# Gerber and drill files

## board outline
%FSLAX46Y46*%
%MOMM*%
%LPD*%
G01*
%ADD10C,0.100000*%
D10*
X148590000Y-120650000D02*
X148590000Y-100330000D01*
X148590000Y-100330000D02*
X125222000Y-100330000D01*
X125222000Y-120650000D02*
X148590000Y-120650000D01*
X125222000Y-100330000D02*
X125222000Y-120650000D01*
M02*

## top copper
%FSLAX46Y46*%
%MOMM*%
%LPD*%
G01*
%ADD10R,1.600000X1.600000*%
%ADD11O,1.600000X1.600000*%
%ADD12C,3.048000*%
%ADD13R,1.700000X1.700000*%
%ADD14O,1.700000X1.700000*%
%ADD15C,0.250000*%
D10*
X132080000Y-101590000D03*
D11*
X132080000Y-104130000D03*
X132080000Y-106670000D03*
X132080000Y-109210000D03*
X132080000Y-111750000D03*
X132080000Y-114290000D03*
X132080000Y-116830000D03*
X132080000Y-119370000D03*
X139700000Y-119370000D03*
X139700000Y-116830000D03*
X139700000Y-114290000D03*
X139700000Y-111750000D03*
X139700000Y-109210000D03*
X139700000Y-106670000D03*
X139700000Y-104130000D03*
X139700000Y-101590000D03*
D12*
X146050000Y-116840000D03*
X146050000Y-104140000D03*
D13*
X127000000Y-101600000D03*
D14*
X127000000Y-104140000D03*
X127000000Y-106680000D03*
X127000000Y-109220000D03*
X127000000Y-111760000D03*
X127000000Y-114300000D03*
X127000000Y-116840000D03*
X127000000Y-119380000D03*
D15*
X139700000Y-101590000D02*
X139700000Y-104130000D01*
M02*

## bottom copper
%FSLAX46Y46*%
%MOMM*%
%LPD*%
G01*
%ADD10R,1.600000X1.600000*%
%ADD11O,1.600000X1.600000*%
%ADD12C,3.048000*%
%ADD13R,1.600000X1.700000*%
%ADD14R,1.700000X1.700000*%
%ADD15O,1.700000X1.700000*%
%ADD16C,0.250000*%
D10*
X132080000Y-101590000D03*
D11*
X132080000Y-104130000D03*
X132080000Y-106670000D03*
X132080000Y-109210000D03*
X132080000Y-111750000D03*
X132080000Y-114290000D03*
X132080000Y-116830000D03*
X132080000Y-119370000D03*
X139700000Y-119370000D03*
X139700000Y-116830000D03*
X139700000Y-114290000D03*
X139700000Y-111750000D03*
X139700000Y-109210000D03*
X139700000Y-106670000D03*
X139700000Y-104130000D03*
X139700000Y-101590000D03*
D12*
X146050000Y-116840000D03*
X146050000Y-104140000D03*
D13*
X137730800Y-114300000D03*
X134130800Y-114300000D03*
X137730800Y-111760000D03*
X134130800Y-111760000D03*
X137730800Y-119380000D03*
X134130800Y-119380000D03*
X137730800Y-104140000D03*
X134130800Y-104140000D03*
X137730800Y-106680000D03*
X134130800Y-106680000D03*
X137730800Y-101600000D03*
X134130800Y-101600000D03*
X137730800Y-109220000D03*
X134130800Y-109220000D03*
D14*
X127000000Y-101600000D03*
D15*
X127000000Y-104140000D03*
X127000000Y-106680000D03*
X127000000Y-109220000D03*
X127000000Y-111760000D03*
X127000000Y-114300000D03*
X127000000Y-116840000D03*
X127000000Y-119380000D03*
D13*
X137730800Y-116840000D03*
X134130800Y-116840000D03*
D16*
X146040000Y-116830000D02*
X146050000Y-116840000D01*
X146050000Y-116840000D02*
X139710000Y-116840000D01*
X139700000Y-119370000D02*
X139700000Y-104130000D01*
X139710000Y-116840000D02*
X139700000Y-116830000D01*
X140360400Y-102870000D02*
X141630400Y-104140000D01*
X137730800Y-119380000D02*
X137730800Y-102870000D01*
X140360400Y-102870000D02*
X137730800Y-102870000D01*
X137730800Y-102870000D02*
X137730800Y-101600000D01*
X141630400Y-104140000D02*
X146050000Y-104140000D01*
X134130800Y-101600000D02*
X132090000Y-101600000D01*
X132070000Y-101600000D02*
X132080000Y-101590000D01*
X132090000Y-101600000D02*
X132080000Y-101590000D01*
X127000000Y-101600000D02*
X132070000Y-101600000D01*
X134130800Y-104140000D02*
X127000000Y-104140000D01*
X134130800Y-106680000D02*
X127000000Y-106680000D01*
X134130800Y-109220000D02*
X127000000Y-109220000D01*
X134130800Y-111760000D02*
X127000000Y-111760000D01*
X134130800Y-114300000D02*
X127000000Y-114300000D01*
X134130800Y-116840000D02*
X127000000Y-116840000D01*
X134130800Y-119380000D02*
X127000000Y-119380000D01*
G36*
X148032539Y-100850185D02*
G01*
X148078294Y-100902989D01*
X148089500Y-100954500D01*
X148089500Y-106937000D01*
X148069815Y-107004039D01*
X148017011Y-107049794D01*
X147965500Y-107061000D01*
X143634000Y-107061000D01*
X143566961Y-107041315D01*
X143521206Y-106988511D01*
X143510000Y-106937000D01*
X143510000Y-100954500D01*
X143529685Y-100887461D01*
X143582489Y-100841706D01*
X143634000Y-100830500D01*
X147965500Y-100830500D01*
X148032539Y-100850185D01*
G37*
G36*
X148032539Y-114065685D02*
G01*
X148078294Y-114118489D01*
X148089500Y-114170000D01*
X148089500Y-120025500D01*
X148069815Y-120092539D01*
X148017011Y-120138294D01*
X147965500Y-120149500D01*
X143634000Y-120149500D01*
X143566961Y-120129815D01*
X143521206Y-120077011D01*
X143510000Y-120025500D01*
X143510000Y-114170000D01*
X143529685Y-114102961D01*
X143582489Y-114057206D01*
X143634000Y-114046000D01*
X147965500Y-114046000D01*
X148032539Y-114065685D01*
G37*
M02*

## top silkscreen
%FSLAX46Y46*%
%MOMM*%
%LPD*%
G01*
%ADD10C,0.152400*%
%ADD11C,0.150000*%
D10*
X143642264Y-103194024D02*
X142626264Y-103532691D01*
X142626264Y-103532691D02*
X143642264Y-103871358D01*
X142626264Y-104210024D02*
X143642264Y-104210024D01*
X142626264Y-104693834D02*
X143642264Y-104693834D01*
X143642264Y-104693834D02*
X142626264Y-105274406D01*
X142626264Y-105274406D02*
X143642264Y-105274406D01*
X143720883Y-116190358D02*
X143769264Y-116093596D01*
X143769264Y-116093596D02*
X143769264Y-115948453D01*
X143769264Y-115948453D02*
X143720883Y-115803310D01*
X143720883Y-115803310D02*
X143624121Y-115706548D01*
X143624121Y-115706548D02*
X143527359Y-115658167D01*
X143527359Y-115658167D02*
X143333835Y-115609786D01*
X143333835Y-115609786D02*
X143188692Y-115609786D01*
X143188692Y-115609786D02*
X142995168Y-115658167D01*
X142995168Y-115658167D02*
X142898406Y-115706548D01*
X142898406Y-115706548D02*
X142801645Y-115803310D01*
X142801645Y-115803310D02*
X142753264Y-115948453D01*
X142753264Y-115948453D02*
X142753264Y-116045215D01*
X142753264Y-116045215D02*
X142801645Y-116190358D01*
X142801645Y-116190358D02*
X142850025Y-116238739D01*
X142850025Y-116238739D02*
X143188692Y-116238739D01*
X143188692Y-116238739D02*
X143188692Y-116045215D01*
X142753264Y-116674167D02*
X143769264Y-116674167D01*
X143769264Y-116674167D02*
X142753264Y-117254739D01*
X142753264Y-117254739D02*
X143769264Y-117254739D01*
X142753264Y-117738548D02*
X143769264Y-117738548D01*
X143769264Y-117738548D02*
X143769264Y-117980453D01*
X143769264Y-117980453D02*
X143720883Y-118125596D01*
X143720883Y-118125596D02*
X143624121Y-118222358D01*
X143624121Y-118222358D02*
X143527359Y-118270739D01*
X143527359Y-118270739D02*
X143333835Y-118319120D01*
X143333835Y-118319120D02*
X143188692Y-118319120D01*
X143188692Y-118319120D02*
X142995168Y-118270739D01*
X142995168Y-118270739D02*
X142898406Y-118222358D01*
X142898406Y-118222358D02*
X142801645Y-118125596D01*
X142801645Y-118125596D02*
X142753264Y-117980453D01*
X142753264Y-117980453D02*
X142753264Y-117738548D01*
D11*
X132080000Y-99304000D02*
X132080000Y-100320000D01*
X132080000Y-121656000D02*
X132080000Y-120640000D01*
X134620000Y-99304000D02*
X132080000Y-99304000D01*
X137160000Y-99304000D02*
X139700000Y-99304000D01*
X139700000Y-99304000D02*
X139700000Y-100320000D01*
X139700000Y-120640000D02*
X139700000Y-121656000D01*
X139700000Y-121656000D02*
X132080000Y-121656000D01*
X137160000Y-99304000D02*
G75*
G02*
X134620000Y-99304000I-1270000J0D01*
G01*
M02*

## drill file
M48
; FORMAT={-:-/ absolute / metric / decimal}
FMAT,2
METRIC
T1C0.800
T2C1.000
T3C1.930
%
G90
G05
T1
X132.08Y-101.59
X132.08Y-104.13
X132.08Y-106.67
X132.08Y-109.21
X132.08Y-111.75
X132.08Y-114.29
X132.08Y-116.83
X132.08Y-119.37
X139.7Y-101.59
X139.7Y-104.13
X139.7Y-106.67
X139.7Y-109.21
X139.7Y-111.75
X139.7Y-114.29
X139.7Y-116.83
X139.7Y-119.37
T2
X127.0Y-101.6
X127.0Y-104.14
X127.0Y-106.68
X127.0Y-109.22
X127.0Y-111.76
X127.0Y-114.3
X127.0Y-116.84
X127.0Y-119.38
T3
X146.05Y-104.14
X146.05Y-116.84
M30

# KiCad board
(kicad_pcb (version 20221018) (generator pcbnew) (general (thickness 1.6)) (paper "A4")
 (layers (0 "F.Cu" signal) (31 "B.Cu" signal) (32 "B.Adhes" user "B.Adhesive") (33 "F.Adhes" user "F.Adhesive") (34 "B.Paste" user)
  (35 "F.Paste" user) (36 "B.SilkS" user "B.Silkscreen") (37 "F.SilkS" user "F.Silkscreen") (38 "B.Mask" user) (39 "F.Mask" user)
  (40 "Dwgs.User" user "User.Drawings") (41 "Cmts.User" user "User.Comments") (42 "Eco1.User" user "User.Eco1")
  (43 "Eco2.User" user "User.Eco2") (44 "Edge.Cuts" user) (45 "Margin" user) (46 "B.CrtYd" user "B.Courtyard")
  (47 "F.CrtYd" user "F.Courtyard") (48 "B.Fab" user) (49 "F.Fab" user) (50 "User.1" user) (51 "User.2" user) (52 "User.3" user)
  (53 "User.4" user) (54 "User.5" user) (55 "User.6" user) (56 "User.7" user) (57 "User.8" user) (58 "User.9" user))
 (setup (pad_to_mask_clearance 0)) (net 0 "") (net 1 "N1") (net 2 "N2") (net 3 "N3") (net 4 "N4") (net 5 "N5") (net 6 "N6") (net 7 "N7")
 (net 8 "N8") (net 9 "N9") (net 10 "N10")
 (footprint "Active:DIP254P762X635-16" (layer "F.Cu") (at 132.08 101.59)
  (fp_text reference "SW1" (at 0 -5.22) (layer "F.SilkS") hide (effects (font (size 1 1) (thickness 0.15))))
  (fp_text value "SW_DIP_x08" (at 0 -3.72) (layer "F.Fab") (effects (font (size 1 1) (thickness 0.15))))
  (fp_line (start 0 -2.286) (end 0 -1.27) (stroke (width 0.15) (type solid)) (layer "F.SilkS"))
  (fp_line (start 0 20.066) (end 0 19.05) (stroke (width 0.15) (type solid)) (layer "F.SilkS"))
  (fp_line (start 2.54 -2.286) (end 0 -2.286) (stroke (width 0.15) (type solid)) (layer "F.SilkS"))
  (fp_line (start 5.08 -2.286) (end 7.62 -2.286) (stroke (width 0.15) (type solid)) (layer "F.SilkS"))
  (fp_line (start 7.62 -2.286) (end 7.62 -1.27) (stroke (width 0.15) (type solid)) (layer "F.SilkS"))
  (fp_line (start 7.62 19.05) (end 7.62 20.066) (stroke (width 0.15) (type solid)) (layer "F.SilkS"))
  (fp_line (start 7.62 20.066) (end 0 20.066) (stroke (width 0.15) (type solid)) (layer "F.SilkS"))
  (fp_arc (start 5.08 -2.286) (mid 3.81 -1.016) (end 2.54 -2.286) (stroke (width 0.15) (type solid)) (layer "F.SilkS"))
  (pad "1" thru_hole rect (at 0 0) (size 1.6 1.6) (drill 0.8) (layers "*.Cu" "*.Mask") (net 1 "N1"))
  (pad "2" thru_hole oval (at 0 2.54) (size 1.6 1.6) (drill 0.8) (layers "*.Cu" "*.Mask") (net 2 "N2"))
  (pad "3" thru_hole oval (at 0 5.08) (size 1.6 1.6) (drill 0.8) (layers "*.Cu" "*.Mask") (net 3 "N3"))
  (pad "4" thru_hole oval (at 0 7.62) (size 1.6 1.6) (drill 0.8) (layers "*.Cu" "*.Mask") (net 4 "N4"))
  (pad "5" thru_hole oval (at 0 10.16) (size 1.6 1.6) (drill 0.8) (layers "*.Cu" "*.Mask") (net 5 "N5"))
  (pad "6" thru_hole oval (at 0 12.7) (size 1.6 1.6) (drill 0.8) (layers "*.Cu" "*.Mask") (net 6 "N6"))
  (pad "7" thru_hole oval (at 0 15.24) (size 1.6 1.6) (drill 0.8) (layers "*.Cu" "*.Mask") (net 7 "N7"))
  (pad "8" thru_hole oval (at 0 17.78) (size 1.6 1.6) (drill 0.8) (layers "*.Cu" "*.Mask") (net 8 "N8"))
  (pad "9" thru_hole oval (at 7.62 17.78) (size 1.6 1.6) (drill 0.8) (layers "*.Cu" "*.Mask") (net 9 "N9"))
  (pad "10" thru_hole oval (at 7.62 15.24) (size 1.6 1.6) (drill 0.8) (layers "*.Cu" "*.Mask") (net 9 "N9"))
  (pad "11" thru_hole oval (at 7.62 12.7) (size 1.6 1.6) (drill 0.8) (layers "*.Cu" "*.Mask") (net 9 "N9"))
  (pad "12" thru_hole oval (at 7.62 10.16) (size 1.6 1.6) (drill 0.8) (layers "*.Cu" "*.Mask") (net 9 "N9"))
  (pad "13" thru_hole oval (at 7.62 7.62) (size 1.6 1.6) (drill 0.8) (layers "*.Cu" "*.Mask") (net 9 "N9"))
  (pad "14" thru_hole oval (at 7.62 5.08) (size 1.6 1.6) (drill 0.8) (layers "*.Cu" "*.Mask") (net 9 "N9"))
  (pad "15" thru_hole oval (at 7.62 2.54) (size 1.6 1.6) (drill 0.8) (layers "*.Cu" "*.Mask") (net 9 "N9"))
  (pad "16" thru_hole oval (at 7.62 0) (size 1.6 1.6) (drill 0.8) (layers "*.Cu" "*.Mask") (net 9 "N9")))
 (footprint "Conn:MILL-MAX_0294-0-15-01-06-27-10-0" (layer "F.Cu") (at 146.05 116.84)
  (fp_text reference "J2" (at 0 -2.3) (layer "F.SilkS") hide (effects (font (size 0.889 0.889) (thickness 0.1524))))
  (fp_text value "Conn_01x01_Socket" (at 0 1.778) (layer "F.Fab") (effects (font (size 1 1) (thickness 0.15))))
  (pad "1" thru_hole circle (at 0 0) (size 3.048 3.048) (drill 1.9304) (layers "*.Cu" "*.Mask") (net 9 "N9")))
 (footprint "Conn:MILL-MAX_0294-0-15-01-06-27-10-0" (layer "F.Cu") (at 146.05 104.14)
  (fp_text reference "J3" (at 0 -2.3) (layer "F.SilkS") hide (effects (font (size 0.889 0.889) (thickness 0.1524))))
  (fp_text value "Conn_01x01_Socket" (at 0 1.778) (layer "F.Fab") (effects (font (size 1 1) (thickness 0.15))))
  (pad "1" thru_hole circle (at 0 0) (size 3.048 3.048) (drill 1.9304) (layers "*.Cu" "*.Mask") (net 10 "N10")))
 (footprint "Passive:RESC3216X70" (layer "B.Cu") (at 135.9308 114.3 180)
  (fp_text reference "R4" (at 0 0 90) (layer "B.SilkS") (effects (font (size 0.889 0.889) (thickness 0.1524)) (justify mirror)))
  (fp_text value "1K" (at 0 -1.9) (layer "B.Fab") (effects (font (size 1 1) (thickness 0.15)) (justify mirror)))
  (pad "1" smd rect (at -1.8 0 180) (size 1.6 1.7) (layers "B.Cu" "B.Paste" "B.Mask") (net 10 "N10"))
  (pad "2" smd rect (at 1.8 0 180) (size 1.6 1.7) (layers "B.Cu" "B.Paste" "B.Mask") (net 6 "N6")))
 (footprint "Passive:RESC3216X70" (layer "B.Cu") (at 135.9308 111.76 180)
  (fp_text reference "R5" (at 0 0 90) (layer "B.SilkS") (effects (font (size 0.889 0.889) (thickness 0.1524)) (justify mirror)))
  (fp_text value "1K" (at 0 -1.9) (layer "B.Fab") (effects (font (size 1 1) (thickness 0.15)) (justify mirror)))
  (pad "1" smd rect (at -1.8 0 180) (size 1.6 1.7) (layers "B.Cu" "B.Paste" "B.Mask") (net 10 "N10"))
  (pad "2" smd rect (at 1.8 0 180) (size 1.6 1.7) (layers "B.Cu" "B.Paste" "B.Mask") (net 5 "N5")))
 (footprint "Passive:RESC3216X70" (layer "B.Cu") (at 135.9308 119.38 180)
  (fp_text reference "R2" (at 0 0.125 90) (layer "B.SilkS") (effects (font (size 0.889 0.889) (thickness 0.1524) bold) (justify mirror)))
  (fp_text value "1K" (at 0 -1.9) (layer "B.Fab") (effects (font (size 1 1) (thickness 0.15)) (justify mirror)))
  (pad "1" smd rect (at -1.8 0 180) (size 1.6 1.7) (layers "B.Cu" "B.Paste" "B.Mask") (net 10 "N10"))
  (pad "2" smd rect (at 1.8 0 180) (size 1.6 1.7) (layers "B.Cu" "B.Paste" "B.Mask") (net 8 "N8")))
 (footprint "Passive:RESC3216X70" (layer "B.Cu") (at 135.9308 104.14 180)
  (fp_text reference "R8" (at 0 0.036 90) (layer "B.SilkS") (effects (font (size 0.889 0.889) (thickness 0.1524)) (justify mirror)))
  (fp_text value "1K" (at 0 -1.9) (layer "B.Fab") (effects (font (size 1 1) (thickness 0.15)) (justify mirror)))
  (pad "1" smd rect (at -1.8 0 180) (size 1.6 1.7) (layers "B.Cu" "B.Paste" "B.Mask") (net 10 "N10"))
  (pad "2" smd rect (at 1.8 0 180) (size 1.6 1.7) (layers "B.Cu" "B.Paste" "B.Mask") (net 2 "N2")))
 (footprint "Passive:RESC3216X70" (layer "B.Cu") (at 135.9308 106.68 180)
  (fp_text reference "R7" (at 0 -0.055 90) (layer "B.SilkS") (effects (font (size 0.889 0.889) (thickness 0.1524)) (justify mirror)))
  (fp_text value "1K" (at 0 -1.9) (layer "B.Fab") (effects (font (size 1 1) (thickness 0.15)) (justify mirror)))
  (pad "1" smd rect (at -1.8 0 180) (size 1.6 1.7) (layers "B.Cu" "B.Paste" "B.Mask") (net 10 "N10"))
  (pad "2" smd rect (at 1.8 0 180) (size 1.6 1.7) (layers "B.Cu" "B.Paste" "B.Mask") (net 3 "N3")))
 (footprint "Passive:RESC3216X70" (layer "B.Cu") (at 135.9308 101.6 180)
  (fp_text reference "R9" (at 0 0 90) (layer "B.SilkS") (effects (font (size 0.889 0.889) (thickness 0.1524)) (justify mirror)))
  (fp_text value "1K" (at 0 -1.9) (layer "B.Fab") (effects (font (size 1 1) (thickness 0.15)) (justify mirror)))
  (pad "1" smd rect (at -1.8 0 180) (size 1.6 1.7) (layers "B.Cu" "B.Paste" "B.Mask") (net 10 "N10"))
  (pad "2" smd rect (at 1.8 0 180) (size 1.6 1.7) (layers "B.Cu" "B.Paste" "B.Mask") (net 1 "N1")))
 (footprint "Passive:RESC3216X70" (layer "B.Cu") (at 135.9308 109.22 180)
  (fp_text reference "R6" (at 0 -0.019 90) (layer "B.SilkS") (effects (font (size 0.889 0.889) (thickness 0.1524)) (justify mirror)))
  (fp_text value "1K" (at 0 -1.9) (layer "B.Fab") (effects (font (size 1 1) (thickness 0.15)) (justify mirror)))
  (pad "1" smd rect (at -1.8 0 180) (size 1.6 1.7) (layers "B.Cu" "B.Paste" "B.Mask") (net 10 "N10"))
  (pad "2" smd rect (at 1.8 0 180) (size 1.6 1.7) (layers "B.Cu" "B.Paste" "B.Mask") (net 4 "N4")))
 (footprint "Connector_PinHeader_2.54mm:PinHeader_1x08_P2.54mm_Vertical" (layer "B.Cu") (at 127 101.6 180)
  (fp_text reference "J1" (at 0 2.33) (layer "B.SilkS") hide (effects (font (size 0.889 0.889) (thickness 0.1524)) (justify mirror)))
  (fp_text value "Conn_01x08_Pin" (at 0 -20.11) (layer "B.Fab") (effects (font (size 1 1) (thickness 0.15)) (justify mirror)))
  (pad "1" thru_hole rect (at 0 0 180) (size 1.7 1.7) (drill 1) (layers "*.Cu" "*.Mask") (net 1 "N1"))
  (pad "2" thru_hole oval (at 0 -2.54 180) (size 1.7 1.7) (drill 1) (layers "*.Cu" "*.Mask") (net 2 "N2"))
  (pad "3" thru_hole oval (at 0 -5.08 180) (size 1.7 1.7) (drill 1) (layers "*.Cu" "*.Mask") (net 3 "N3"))
  (pad "4" thru_hole oval (at 0 -7.62 180) (size 1.7 1.7) (drill 1) (layers "*.Cu" "*.Mask") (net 4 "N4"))
  (pad "5" thru_hole oval (at 0 -10.16 180) (size 1.7 1.7) (drill 1) (layers "*.Cu" "*.Mask") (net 5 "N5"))
  (pad "6" thru_hole oval (at 0 -12.7 180) (size 1.7 1.7) (drill 1) (layers "*.Cu" "*.Mask") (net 6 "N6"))
  (pad "7" thru_hole oval (at 0 -15.24 180) (size 1.7 1.7) (drill 1) (layers "*.Cu" "*.Mask") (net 7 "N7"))
  (pad "8" thru_hole oval (at 0 -17.78 180) (size 1.7 1.7) (drill 1) (layers "*.Cu" "*.Mask") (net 8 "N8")))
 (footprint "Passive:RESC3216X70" (layer "B.Cu") (at 135.9308 116.84 180)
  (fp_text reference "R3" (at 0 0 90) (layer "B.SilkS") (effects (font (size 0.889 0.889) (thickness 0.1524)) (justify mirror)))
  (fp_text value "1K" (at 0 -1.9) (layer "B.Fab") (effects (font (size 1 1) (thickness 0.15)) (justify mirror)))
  (pad "1" smd rect (at -1.8 0 180) (size 1.6 1.7) (layers "B.Cu" "B.Paste" "B.Mask") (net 10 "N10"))
  (pad "2" smd rect (at 1.8 0 180) (size 1.6 1.7) (layers "B.Cu" "B.Paste" "B.Mask") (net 7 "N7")))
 (gr_line (start 148.59 120.65) (end 148.59 100.33) (stroke (width 0.1) (type default)) (layer "Edge.Cuts"))
 (gr_line (start 148.59 100.33) (end 125.222 100.33) (stroke (width 0.1) (type default)) (layer "Edge.Cuts"))
 (gr_line (start 125.222 120.65) (end 148.59 120.65) (stroke (width 0.1) (type default)) (layer "Edge.Cuts"))
 (gr_line (start 125.222 100.33) (end 125.222 120.65) (stroke (width 0.1) (type default)) (layer "Edge.Cuts"))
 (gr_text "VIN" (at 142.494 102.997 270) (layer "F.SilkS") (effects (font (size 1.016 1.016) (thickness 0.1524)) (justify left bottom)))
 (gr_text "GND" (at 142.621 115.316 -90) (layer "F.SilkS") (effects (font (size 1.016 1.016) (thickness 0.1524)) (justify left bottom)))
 (segment (start 139.7 101.59) (end 139.7 104.13) (width 0.25) (layer "F.Cu") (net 9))
 (segment (start 146.04 116.83) (end 146.05 116.84) (width 0.25) (layer "B.Cu") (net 9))
 (segment (start 146.05 116.84) (end 139.71 116.84) (width 0.25) (layer "B.Cu") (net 9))
 (segment (start 139.7 119.37) (end 139.7 104.13) (width 0.25) (layer "B.Cu") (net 9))
 (segment (start 139.71 116.84) (end 139.7 116.83) (width 0.25) (layer "B.Cu") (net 9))
 (segment (start 140.3604 102.87) (end 141.6304 104.14) (width 0.25) (layer "B.Cu") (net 10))
 (segment (start 137.7308 119.38) (end 137.7308 102.87) (width 0.25) (layer "B.Cu") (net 10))
 (segment (start 140.3604 102.87) (end 137.7308 102.87) (width 0.25) (layer "B.Cu") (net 10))
 (segment (start 137.7308 102.87) (end 137.7308 101.6) (width 0.25) (layer "B.Cu") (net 10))
 (segment (start 141.6304 104.14) (end 146.05 104.14) (width 0.25) (layer "B.Cu") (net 10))
 (segment (start 134.1308 101.6) (end 132.09 101.6) (width 0.25) (layer "B.Cu") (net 1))
 (segment (start 132.07 101.6) (end 132.08 101.59) (width 0.25) (layer "B.Cu") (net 1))
 (segment (start 132.09 101.6) (end 132.08 101.59) (width 0.25) (layer "B.Cu") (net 1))
 (segment (start 127 101.6) (end 132.07 101.6) (width 0.25) (layer "B.Cu") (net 1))
 (segment (start 134.1308 104.14) (end 127 104.14) (width 0.25) (layer "B.Cu") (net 2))
 (segment (start 134.1308 106.68) (end 127 106.68) (width 0.25) (layer "B.Cu") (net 3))
 (segment (start 134.1308 109.22) (end 127 109.22) (width 0.25) (layer "B.Cu") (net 4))
 (segment (start 134.1308 111.76) (end 127 111.76) (width 0.25) (layer "B.Cu") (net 5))
 (segment (start 134.1308 114.3) (end 127 114.3) (width 0.25) (layer "B.Cu") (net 6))
 (segment (start 134.1308 116.84) (end 127 116.84) (width 0.25) (layer "B.Cu") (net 7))
 (segment (start 134.1308 119.38) (end 127 119.38) (width 0.25) (layer "B.Cu") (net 8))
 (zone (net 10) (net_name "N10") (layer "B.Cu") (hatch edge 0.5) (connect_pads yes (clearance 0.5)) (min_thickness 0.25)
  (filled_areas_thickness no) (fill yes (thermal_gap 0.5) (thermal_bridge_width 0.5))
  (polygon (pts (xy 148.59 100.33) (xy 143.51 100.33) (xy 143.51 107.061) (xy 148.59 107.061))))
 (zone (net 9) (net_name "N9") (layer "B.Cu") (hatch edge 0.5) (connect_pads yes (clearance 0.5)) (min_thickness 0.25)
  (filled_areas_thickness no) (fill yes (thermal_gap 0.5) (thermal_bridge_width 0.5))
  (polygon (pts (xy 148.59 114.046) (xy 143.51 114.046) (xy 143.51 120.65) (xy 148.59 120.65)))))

